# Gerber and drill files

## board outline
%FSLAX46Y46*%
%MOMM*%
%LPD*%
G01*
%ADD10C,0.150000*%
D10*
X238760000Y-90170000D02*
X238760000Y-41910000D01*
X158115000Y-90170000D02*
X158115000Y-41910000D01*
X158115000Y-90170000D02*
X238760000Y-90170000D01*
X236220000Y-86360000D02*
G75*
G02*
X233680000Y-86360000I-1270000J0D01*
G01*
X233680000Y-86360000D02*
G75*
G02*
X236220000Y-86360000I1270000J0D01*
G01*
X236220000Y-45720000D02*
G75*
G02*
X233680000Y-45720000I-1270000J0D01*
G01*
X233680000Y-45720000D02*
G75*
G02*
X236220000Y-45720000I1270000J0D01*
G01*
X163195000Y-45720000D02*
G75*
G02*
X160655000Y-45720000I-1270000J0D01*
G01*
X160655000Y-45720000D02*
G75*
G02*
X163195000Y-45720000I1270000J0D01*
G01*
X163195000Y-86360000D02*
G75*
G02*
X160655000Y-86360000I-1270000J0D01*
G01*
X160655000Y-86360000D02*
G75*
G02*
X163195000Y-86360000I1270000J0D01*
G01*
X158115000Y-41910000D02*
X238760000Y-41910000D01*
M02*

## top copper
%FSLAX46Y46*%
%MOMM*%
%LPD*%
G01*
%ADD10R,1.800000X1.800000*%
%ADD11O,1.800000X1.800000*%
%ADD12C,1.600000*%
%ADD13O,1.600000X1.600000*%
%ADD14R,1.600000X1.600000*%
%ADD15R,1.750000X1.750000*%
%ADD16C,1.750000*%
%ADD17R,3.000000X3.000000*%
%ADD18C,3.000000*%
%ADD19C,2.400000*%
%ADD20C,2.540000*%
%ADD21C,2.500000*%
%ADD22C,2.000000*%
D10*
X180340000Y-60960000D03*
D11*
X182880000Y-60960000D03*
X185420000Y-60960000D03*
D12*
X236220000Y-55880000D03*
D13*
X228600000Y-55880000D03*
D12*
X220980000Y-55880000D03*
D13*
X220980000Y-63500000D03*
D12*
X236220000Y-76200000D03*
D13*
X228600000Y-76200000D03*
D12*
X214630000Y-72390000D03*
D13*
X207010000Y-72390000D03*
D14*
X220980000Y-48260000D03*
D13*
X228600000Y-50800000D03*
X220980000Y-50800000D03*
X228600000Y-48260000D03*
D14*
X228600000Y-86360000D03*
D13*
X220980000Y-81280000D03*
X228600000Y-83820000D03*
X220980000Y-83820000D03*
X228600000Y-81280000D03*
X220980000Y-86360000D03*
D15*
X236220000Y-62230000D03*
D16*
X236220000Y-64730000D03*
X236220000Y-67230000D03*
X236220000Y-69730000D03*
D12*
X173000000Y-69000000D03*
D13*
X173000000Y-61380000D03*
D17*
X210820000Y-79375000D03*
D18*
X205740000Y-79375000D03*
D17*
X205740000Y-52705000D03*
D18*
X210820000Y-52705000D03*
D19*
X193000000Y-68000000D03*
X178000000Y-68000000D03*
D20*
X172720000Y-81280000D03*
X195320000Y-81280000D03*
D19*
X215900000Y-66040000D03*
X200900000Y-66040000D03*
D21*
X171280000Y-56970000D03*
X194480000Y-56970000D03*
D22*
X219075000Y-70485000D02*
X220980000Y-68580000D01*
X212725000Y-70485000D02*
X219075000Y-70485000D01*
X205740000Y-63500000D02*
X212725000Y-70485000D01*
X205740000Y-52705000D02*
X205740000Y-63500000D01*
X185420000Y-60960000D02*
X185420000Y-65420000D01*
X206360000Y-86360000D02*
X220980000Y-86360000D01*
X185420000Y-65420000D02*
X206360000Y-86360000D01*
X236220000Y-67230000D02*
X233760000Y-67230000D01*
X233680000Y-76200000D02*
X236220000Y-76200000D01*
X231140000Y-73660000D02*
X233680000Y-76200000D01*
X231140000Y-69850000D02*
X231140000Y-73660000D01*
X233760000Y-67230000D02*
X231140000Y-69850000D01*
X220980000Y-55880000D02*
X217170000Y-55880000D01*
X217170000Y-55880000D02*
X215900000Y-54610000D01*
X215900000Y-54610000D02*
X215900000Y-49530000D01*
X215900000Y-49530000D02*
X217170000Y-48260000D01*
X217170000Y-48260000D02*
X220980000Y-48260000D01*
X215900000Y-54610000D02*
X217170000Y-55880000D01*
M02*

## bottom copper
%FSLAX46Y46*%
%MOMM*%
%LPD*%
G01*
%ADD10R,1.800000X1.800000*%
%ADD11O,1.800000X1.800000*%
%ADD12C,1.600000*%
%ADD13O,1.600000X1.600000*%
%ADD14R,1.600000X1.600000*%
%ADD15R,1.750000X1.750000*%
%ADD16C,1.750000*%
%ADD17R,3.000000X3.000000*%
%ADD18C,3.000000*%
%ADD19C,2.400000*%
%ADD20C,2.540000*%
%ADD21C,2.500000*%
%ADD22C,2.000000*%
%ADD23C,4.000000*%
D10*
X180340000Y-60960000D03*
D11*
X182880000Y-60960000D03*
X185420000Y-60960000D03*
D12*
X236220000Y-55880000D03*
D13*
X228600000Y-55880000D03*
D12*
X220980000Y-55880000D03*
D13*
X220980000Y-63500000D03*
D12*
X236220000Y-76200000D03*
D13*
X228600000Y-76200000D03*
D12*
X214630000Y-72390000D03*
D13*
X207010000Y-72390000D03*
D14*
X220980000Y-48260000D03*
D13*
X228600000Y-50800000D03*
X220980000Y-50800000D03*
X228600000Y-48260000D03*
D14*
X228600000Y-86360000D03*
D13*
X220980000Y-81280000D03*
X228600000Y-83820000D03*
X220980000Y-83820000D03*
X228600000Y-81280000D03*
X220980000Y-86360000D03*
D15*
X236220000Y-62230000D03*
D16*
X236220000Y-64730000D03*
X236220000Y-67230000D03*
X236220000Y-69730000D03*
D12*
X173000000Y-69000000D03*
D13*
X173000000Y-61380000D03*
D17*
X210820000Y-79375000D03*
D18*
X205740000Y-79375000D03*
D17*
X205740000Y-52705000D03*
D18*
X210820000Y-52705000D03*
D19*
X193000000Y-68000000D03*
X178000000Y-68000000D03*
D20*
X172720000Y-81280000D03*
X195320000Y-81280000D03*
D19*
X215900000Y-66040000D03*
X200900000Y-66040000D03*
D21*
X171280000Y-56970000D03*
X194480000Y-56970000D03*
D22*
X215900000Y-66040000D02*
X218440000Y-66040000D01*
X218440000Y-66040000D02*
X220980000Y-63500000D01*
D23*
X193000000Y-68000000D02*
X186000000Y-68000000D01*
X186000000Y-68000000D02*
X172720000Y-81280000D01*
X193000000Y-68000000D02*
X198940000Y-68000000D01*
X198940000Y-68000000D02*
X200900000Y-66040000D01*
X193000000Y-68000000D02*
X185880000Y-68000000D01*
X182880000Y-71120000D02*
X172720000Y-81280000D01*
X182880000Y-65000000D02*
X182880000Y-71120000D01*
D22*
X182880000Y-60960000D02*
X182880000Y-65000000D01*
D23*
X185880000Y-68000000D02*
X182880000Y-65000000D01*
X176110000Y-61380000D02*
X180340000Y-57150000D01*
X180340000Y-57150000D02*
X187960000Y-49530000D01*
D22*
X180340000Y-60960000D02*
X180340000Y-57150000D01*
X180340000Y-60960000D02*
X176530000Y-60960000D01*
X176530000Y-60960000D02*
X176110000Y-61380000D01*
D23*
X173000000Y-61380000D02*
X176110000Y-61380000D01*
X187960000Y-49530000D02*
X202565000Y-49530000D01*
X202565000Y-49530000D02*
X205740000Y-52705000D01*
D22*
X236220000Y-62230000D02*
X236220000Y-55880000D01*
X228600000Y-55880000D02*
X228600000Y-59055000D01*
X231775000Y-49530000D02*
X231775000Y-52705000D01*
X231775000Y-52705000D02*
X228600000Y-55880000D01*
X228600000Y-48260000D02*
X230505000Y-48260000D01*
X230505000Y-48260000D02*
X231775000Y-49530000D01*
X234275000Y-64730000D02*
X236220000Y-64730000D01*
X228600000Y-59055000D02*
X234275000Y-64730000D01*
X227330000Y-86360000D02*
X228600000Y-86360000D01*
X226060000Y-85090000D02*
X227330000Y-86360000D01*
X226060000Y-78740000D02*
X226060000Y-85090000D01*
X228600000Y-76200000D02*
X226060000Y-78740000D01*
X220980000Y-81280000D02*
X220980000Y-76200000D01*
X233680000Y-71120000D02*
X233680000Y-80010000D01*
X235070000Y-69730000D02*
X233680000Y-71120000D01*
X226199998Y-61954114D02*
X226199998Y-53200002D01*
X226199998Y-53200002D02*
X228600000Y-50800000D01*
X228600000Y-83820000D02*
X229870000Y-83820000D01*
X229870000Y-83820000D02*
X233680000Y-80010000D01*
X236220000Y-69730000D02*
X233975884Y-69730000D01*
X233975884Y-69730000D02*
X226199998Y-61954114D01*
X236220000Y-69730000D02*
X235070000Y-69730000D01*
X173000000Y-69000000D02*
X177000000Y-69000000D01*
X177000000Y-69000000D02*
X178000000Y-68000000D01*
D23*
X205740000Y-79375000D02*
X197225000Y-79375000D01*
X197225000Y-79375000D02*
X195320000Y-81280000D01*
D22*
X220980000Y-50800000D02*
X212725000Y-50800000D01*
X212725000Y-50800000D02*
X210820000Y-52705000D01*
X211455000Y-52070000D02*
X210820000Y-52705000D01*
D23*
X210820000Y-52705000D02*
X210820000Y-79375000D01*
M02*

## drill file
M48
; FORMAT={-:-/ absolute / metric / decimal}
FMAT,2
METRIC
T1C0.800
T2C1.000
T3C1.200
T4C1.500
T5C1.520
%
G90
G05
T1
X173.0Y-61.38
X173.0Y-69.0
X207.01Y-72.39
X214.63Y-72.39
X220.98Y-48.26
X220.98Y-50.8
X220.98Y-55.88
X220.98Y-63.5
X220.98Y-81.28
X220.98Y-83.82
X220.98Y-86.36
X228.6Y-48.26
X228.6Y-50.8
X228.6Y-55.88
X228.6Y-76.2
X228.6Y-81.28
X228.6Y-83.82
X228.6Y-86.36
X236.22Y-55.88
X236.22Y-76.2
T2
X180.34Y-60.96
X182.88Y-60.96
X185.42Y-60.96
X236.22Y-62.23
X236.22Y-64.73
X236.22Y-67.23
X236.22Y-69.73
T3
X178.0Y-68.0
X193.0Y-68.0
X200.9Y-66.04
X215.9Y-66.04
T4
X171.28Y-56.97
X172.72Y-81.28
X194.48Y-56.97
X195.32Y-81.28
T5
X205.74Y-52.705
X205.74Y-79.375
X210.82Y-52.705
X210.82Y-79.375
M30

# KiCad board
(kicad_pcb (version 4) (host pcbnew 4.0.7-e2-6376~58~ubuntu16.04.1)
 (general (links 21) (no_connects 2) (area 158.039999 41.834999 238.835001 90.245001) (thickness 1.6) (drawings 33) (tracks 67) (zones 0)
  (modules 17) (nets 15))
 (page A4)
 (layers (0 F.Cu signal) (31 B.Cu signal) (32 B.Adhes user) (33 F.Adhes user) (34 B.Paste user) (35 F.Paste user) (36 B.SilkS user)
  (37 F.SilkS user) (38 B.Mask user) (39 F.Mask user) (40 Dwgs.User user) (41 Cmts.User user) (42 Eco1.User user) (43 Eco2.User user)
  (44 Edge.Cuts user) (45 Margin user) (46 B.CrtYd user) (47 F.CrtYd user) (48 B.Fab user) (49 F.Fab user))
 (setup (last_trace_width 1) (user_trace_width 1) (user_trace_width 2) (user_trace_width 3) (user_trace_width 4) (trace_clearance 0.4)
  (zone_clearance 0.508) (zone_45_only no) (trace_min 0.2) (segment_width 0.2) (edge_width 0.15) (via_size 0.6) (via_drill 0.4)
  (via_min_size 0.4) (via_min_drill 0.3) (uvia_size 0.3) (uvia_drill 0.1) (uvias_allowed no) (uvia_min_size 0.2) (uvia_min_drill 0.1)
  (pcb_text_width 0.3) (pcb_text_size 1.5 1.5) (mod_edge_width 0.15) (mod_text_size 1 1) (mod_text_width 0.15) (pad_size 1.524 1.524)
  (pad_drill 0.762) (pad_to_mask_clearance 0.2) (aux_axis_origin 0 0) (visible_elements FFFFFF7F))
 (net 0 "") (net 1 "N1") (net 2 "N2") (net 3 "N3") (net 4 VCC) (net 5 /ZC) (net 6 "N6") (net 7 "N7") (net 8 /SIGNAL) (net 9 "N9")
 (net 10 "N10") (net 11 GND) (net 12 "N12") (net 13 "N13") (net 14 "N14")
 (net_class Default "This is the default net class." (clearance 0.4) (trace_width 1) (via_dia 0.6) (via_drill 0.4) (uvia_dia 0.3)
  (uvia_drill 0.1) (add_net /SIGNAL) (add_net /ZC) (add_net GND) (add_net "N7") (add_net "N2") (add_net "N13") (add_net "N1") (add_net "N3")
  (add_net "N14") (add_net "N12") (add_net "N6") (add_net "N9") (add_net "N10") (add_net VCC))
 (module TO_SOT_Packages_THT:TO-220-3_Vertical (layer F.Cu) (at 180.34 60.96)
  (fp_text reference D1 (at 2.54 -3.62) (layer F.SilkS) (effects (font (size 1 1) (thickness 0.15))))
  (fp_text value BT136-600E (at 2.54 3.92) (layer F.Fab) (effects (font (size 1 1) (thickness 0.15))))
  (pad 1 thru_hole rect (at 0 0) (size 1.8 1.8) (drill 1) (layers *.Cu *.Mask) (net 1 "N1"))
  (pad 2 thru_hole oval (at 2.54 0) (size 1.8 1.8) (drill 1) (layers *.Cu *.Mask) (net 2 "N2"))
  (pad 3 thru_hole oval (at 5.08 0) (size 1.8 1.8) (drill 1) (layers *.Cu *.Mask) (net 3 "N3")))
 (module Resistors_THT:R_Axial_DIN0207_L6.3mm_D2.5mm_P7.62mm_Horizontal (layer F.Cu) (at 236.22 55.88 180)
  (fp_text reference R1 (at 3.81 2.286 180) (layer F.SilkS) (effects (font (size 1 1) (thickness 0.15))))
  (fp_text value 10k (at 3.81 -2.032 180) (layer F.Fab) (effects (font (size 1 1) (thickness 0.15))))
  (pad 1 thru_hole circle (at 0 0 180) (size 1.6 1.6) (drill 0.8) (layers *.Cu *.Mask) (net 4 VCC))
  (pad 2 thru_hole oval (at 7.62 0 180) (size 1.6 1.6) (drill 0.8) (layers *.Cu *.Mask) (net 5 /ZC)))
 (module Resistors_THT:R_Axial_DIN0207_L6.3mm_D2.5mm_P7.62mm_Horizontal (layer F.Cu) (at 220.98 55.88 270)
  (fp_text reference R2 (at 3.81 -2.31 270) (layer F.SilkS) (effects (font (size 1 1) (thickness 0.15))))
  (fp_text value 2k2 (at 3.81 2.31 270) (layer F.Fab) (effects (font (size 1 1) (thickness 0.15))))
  (pad 1 thru_hole circle (at 0 0 270) (size 1.6 1.6) (drill 0.8) (layers *.Cu *.Mask) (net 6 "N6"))
  (pad 2 thru_hole oval (at 7.62 0 270) (size 1.6 1.6) (drill 0.8) (layers *.Cu *.Mask) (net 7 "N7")))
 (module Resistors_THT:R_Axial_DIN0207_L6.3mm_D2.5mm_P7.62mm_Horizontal (layer F.Cu) (at 236.22 76.2 180)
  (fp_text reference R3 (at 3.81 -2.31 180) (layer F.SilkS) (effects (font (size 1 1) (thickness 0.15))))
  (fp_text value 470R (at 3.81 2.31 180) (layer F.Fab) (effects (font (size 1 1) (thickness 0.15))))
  (pad 1 thru_hole circle (at 0 0 180) (size 1.6 1.6) (drill 0.8) (layers *.Cu *.Mask) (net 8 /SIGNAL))
  (pad 2 thru_hole oval (at 7.62 0 180) (size 1.6 1.6) (drill 0.8) (layers *.Cu *.Mask) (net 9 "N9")))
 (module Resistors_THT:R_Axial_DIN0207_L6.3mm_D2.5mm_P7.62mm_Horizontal (layer F.Cu) (at 214.63 72.39 180)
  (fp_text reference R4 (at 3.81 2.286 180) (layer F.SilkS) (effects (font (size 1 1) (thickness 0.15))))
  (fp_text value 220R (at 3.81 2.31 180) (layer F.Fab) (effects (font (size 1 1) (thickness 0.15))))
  (pad 1 thru_hole circle (at 0 0 180) (size 1.6 1.6) (drill 0.8) (layers *.Cu *.Mask) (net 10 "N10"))
  (pad 2 thru_hole oval (at 7.62 0 180) (size 1.6 1.6) (drill 0.8) (layers *.Cu *.Mask) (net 2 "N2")))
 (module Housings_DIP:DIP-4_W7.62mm (layer F.Cu) (at 220.98 48.26)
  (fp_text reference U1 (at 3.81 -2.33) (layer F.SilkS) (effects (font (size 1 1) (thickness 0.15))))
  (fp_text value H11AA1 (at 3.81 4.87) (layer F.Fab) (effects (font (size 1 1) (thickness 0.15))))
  (pad 1 thru_hole rect (at 0 0) (size 1.6 1.6) (drill 0.8) (layers *.Cu *.Mask) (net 6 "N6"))
  (pad 3 thru_hole oval (at 7.62 2.54) (size 1.6 1.6) (drill 0.8) (layers *.Cu *.Mask) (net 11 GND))
  (pad 2 thru_hole oval (at 0 2.54) (size 1.6 1.6) (drill 0.8) (layers *.Cu *.Mask) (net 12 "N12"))
  (pad 4 thru_hole oval (at 7.62 0) (size 1.6 1.6) (drill 0.8) (layers *.Cu *.Mask) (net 5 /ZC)))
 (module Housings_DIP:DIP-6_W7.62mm (layer F.Cu) (at 228.6 86.36 180)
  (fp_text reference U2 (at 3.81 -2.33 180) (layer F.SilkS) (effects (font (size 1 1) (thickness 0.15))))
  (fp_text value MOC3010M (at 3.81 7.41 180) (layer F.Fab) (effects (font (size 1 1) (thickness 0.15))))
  (pad 1 thru_hole rect (at 0 0 180) (size 1.6 1.6) (drill 0.8) (layers *.Cu *.Mask) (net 9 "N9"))
  (pad 4 thru_hole oval (at 7.62 5.08 180) (size 1.6 1.6) (drill 0.8) (layers *.Cu *.Mask) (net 10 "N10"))
  (pad 2 thru_hole oval (at 0 2.54 180) (size 1.6 1.6) (drill 0.8) (layers *.Cu *.Mask) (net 11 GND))
  (pad 5 thru_hole oval (at 7.62 2.54 180) (size 1.6 1.6) (drill 0.8) (layers *.Cu *.Mask))
  (pad 3 thru_hole oval (at 0 5.08 180) (size 1.6 1.6) (drill 0.8) (layers *.Cu *.Mask))
  (pad 6 thru_hole oval (at 7.62 0 180) (size 1.6 1.6) (drill 0.8) (layers *.Cu *.Mask) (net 3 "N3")))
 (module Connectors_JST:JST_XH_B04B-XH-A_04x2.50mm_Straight (layer F.Cu) (at 236.22 62.23 270)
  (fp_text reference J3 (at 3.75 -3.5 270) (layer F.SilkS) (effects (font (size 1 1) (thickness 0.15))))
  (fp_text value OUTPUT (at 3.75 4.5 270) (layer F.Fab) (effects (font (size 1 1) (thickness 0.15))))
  (pad 1 thru_hole rect (at 0 0 270) (size 1.75 1.75) (drill 1) (layers *.Cu *.Mask) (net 4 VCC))
  (pad 2 thru_hole circle (at 2.5 0 270) (size 1.75 1.75) (drill 1) (layers *.Cu *.Mask) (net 5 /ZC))
  (pad 3 thru_hole circle (at 5 0 270) (size 1.75 1.75) (drill 1) (layers *.Cu *.Mask) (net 8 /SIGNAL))
  (pad 4 thru_hole circle (at 7.5 0 270) (size 1.75 1.75) (drill 1) (layers *.Cu *.Mask) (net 11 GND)))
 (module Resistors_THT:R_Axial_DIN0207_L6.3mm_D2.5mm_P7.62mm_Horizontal (layer F.Cu) (at 173 69 90)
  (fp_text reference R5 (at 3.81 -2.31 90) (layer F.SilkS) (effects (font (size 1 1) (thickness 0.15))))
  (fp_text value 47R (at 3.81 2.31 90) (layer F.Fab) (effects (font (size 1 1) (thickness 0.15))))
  (pad 1 thru_hole circle (at 0 0 90) (size 1.6 1.6) (drill 0.8) (layers *.Cu *.Mask) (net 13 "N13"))
  (pad 2 thru_hole oval (at 7.62 0 90) (size 1.6 1.6) (drill 0.8) (layers *.Cu *.Mask) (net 1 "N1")))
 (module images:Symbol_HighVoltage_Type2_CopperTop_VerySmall (layer F.Cu) (at 163.83 74.93 270)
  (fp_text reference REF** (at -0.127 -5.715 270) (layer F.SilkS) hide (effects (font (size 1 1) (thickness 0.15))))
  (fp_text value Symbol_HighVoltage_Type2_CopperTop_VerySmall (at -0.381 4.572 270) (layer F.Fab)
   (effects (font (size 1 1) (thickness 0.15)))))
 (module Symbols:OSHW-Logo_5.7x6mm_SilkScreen (layer F.Cu) (at 216.916 76.708)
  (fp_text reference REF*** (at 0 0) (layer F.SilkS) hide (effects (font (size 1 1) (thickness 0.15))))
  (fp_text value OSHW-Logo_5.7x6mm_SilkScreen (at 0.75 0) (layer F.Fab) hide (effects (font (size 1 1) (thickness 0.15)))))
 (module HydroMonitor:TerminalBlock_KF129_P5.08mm (layer F.Cu) (at 210.82 79.375 180)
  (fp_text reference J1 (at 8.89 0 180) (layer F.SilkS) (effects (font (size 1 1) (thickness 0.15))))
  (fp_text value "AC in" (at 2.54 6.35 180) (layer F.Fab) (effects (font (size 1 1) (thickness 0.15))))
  (pad 1 thru_hole rect (at 0 0 180) (size 3 3) (drill 1.52) (layers *.Cu *.Mask) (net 12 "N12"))
  (pad 2 thru_hole circle (at 5.08 0 180) (size 3 3) (drill 1.52) (layers *.Cu *.Mask) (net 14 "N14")))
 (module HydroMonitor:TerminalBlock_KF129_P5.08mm (layer F.Cu) (at 205.74 52.705)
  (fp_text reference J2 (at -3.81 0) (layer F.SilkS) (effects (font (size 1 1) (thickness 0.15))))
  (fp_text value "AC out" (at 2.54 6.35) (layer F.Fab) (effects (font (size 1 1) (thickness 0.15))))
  (pad 1 thru_hole rect (at 0 0) (size 3 3) (drill 1.52) (layers *.Cu *.Mask) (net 1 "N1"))
  (pad 2 thru_hole circle (at 5.08 0) (size 3 3) (drill 1.52) (layers *.Cu *.Mask) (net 12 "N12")))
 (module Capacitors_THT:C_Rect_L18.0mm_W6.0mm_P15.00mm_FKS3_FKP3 (layer F.Cu) (at 193 68 180)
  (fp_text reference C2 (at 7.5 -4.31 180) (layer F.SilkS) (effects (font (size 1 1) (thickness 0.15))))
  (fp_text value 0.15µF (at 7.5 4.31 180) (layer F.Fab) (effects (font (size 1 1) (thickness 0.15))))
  (pad 1 thru_hole circle (at 0 0 180) (size 2.4 2.4) (drill 1.2) (layers *.Cu *.Mask) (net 2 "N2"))
  (pad 2 thru_hole circle (at 15 0 180) (size 2.4 2.4) (drill 1.2) (layers *.Cu *.Mask) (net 13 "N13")))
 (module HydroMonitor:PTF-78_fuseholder (layer F.Cu) (at 172.72 81.28)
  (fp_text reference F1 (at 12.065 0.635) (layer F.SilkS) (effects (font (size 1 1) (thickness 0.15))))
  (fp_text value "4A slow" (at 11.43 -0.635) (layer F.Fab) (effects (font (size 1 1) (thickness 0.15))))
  (pad 1 thru_hole circle (at 0 0) (size 2.54 2.54) (drill 1.5) (layers *.Cu *.Mask) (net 2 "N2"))
  (pad 2 thru_hole circle (at 22.6 0) (size 2.54 2.54) (drill 1.5) (layers *.Cu *.Mask) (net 14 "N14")))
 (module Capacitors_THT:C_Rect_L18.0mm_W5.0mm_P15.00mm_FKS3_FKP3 (layer F.Cu) (at 215.9 66.04 180)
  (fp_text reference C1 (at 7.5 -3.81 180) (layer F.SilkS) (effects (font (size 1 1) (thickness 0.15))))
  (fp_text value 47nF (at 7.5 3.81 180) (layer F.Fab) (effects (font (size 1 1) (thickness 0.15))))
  (pad 1 thru_hole circle (at 0 0 180) (size 2.4 2.4) (drill 1.2) (layers *.Cu *.Mask) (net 7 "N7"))
  (pad 2 thru_hole circle (at 15 0 180) (size 2.4 2.4) (drill 1.2) (layers *.Cu *.Mask) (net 2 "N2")))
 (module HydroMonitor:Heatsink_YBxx (layer F.Cu) (at 182.88 58.42 180)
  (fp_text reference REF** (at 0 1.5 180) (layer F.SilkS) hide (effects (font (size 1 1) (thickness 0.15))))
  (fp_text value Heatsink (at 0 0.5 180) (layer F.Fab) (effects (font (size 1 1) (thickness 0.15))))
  (pad "" thru_hole circle (at 11.6 1.45 180) (size 2.5 2.5) (drill 1.5) (layers *.Cu *.Mask))
  (pad "" thru_hole circle (at -11.6 1.45 180) (size 2.5 2.5) (drill 1.5) (layers *.Cu *.Mask)))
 (gr_line (start 238.76 90.17) (end 238.76 41.91) (angle 90) (layer Edge.Cuts) (width 0.15))
 (gr_line (start 158.115 90.17) (end 158.115 41.91) (angle 90) (layer Edge.Cuts) (width 0.15))
 (gr_line (start 158.115 90.17) (end 238.76 90.17) (angle 90) (layer Edge.Cuts) (width 0.15))
 (gr_circle (center 234.95 86.36) (end 236.22 86.36) (layer Edge.Cuts) (width 0.15))
 (gr_circle (center 234.95 45.72) (end 236.22 45.72) (layer Edge.Cuts) (width 0.15))
 (gr_circle (center 161.925 45.72) (end 161.925 44.45) (layer Edge.Cuts) (width 0.15))
 (gr_circle (center 161.925 86.36) (end 161.925 87.63) (layer Edge.Cuts) (width 0.15))
 (gr_line (start 158.115 41.91) (end 238.76 41.91) (angle 90) (layer Edge.Cuts) (width 0.15))
 (segment (start 215.9 66.04) (end 218.44 66.04) (width 2) (layer B.Cu) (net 7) (status 10))
 (segment (start 218.44 66.04) (end 220.98 63.5) (width 2) (layer B.Cu) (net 7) (status 20))
 (segment (start 193 68) (end 186 68) (width 4) (layer B.Cu) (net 2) (status 10))
 (segment (start 186 68) (end 172.72 81.28) (width 4) (layer B.Cu) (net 2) (status 20))
 (segment (start 193 68) (end 198.94 68) (width 4) (layer B.Cu) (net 2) (status 10))
 (segment (start 198.94 68) (end 200.9 66.04) (width 4) (layer B.Cu) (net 2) (status 20))
 (segment (start 193 68) (end 185.88 68) (width 4) (layer B.Cu) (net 2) (status 10))
 (segment (start 182.88 71.12) (end 172.72 81.28) (width 4) (layer B.Cu) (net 2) (status 20))
 (segment (start 182.88 65) (end 182.88 71.12) (width 4) (layer B.Cu) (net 2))
 (segment (start 182.88 60.96) (end 182.88 65) (width 2) (layer B.Cu) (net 2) (status 10))
 (segment (start 185.88 68) (end 182.88 65) (width 4) (layer B.Cu) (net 2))
 (segment (start 219.075 70.485) (end 220.98 68.58) (width 2) (layer F.Cu) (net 1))
 (segment (start 212.725 70.485) (end 219.075 70.485) (width 2) (layer F.Cu) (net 1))
 (segment (start 205.74 63.5) (end 212.725 70.485) (width 2) (layer F.Cu) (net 1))
 (segment (start 205.74 52.705) (end 205.74 63.5) (width 2) (layer F.Cu) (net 1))
 (segment (start 176.11 61.38) (end 180.34 57.15) (width 4) (layer B.Cu) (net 1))
 (segment (start 180.34 57.15) (end 187.96 49.53) (width 4) (layer B.Cu) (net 1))
 (segment (start 180.34 60.96) (end 180.34 57.15) (width 2) (layer B.Cu) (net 1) (status 10))
 (segment (start 180.34 60.96) (end 176.53 60.96) (width 2) (layer B.Cu) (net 1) (status 10))
 (segment (start 176.53 60.96) (end 176.11 61.38) (width 2) (layer B.Cu) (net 1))
 (segment (start 173 61.38) (end 176.11 61.38) (width 4) (layer B.Cu) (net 1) (status 10))
 (segment (start 187.96 49.53) (end 202.565 49.53) (width 4) (layer B.Cu) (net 1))
 (segment (start 202.565 49.53) (end 205.74 52.705) (width 4) (layer B.Cu) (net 1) (status 20))
 (segment (start 185.42 60.96) (end 185.42 65.42) (width 2) (layer F.Cu) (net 3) (status 10))
 (segment (start 206.36 86.36) (end 220.98 86.36) (width 2) (layer F.Cu) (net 3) (status 20))
 (segment (start 185.42 65.42) (end 206.36 86.36) (width 2) (layer F.Cu) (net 3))
 (segment (start 236.22 62.23) (end 236.22 55.88) (width 2) (layer B.Cu) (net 4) (status 30))
 (segment (start 228.6 55.88) (end 228.6 59.055) (width 2) (layer B.Cu) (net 5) (status 10))
 (segment (start 231.775 49.53) (end 231.775 52.705) (width 2) (layer B.Cu) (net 5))
 (segment (start 231.775 52.705) (end 228.6 55.88) (width 2) (layer B.Cu) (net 5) (status 20))
 (segment (start 228.6 48.26) (end 230.505 48.26) (width 2) (layer B.Cu) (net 5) (status 10))
 (segment (start 230.505 48.26) (end 231.775 49.53) (width 2) (layer B.Cu) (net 5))
 (segment (start 234.275 64.73) (end 236.22 64.73) (width 2) (layer B.Cu) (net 5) (status 20))
 (segment (start 228.6 59.055) (end 234.275 64.73) (width 2) (layer B.Cu) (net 5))
 (segment (start 236.22 67.23) (end 233.76 67.23) (width 2) (layer F.Cu) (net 8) (status 10))
 (segment (start 233.68 76.2) (end 236.22 76.2) (width 2) (layer F.Cu) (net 8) (status 20))
 (segment (start 231.14 73.66) (end 233.68 76.2) (width 2) (layer F.Cu) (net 8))
 (segment (start 231.14 69.85) (end 231.14 73.66) (width 2) (layer F.Cu) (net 8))
 (segment (start 233.76 67.23) (end 231.14 69.85) (width 2) (layer F.Cu) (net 8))
 (segment (start 227.33 86.36) (end 228.6 86.36) (width 2) (layer B.Cu) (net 9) (status 20))
 (segment (start 226.06 85.09) (end 227.33 86.36) (width 2) (layer B.Cu) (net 9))
 (segment (start 226.06 78.74) (end 226.06 85.09) (width 2) (layer B.Cu) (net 9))
 (segment (start 228.6 76.2) (end 226.06 78.74) (width 2) (layer B.Cu) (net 9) (status 10))
 (segment (start 220.98 81.28) (end 220.98 76.2) (width 2) (layer B.Cu) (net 10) (status 30))
 (segment (start 233.68 71.12) (end 233.68 80.01) (width 2) (layer B.Cu) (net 11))
 (segment (start 235.07 69.73) (end 233.68 71.12) (width 2) (layer B.Cu) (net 11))
 (segment (start 226.199998 61.954114) (end 226.199998 53.200002) (width 2) (layer B.Cu) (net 11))
 (segment (start 226.199998 53.200002) (end 228.6 50.8) (width 2) (layer B.Cu) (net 11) (status 20))
 (segment (start 228.6 83.82) (end 229.87 83.82) (width 2) (layer B.Cu) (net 11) (status 10))
 (segment (start 229.87 83.82) (end 233.68 80.01) (width 2) (layer B.Cu) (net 11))
 (segment (start 236.22 69.73) (end 233.975884 69.73) (width 2) (layer B.Cu) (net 11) (status 10))
 (segment (start 233.975884 69.73) (end 226.199998 61.954114) (width 2) (layer B.Cu) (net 11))
 (segment (start 236.22 69.73) (end 235.07 69.73) (width 2) (layer B.Cu) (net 11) (status 10))
 (segment (start 173 69) (end 177 69) (width 2) (layer B.Cu) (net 13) (status 10))
 (segment (start 177 69) (end 178 68) (width 2) (layer B.Cu) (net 13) (status 20))
 (segment (start 205.74 79.375) (end 197.225 79.375) (width 4) (layer B.Cu) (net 14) (status 10))
 (segment (start 197.225 79.375) (end 195.32 81.28) (width 4) (layer B.Cu) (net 14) (status 20))
 (segment (start 220.98 50.8) (end 212.725 50.8) (width 2) (layer B.Cu) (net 12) (status 10))
 (segment (start 212.725 50.8) (end 210.82 52.705) (width 2) (layer B.Cu) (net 12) (status 20))
 (segment (start 211.455 52.07) (end 210.82 52.705) (width 2) (layer B.Cu) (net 12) (status 30))
 (segment (start 210.82 52.705) (end 210.82 79.375) (width 4) (layer B.Cu) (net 12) (status 30))
 (segment (start 220.98 55.88) (end 217.17 55.88) (width 2) (layer F.Cu) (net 6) (status 10))
 (segment (start 217.17 55.88) (end 215.9 54.61) (width 2) (layer F.Cu) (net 6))
 (segment (start 215.9 54.61) (end 215.9 49.53) (width 2) (layer F.Cu) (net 6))
 (segment (start 215.9 49.53) (end 217.17 48.26) (width 2) (layer F.Cu) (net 6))
 (segment (start 217.17 48.26) (end 220.98 48.26) (width 2) (layer F.Cu) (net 6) (status 20))
 (segment (start 215.9 54.61) (end 217.17 55.88) (width 2) (layer F.Cu) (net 6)))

